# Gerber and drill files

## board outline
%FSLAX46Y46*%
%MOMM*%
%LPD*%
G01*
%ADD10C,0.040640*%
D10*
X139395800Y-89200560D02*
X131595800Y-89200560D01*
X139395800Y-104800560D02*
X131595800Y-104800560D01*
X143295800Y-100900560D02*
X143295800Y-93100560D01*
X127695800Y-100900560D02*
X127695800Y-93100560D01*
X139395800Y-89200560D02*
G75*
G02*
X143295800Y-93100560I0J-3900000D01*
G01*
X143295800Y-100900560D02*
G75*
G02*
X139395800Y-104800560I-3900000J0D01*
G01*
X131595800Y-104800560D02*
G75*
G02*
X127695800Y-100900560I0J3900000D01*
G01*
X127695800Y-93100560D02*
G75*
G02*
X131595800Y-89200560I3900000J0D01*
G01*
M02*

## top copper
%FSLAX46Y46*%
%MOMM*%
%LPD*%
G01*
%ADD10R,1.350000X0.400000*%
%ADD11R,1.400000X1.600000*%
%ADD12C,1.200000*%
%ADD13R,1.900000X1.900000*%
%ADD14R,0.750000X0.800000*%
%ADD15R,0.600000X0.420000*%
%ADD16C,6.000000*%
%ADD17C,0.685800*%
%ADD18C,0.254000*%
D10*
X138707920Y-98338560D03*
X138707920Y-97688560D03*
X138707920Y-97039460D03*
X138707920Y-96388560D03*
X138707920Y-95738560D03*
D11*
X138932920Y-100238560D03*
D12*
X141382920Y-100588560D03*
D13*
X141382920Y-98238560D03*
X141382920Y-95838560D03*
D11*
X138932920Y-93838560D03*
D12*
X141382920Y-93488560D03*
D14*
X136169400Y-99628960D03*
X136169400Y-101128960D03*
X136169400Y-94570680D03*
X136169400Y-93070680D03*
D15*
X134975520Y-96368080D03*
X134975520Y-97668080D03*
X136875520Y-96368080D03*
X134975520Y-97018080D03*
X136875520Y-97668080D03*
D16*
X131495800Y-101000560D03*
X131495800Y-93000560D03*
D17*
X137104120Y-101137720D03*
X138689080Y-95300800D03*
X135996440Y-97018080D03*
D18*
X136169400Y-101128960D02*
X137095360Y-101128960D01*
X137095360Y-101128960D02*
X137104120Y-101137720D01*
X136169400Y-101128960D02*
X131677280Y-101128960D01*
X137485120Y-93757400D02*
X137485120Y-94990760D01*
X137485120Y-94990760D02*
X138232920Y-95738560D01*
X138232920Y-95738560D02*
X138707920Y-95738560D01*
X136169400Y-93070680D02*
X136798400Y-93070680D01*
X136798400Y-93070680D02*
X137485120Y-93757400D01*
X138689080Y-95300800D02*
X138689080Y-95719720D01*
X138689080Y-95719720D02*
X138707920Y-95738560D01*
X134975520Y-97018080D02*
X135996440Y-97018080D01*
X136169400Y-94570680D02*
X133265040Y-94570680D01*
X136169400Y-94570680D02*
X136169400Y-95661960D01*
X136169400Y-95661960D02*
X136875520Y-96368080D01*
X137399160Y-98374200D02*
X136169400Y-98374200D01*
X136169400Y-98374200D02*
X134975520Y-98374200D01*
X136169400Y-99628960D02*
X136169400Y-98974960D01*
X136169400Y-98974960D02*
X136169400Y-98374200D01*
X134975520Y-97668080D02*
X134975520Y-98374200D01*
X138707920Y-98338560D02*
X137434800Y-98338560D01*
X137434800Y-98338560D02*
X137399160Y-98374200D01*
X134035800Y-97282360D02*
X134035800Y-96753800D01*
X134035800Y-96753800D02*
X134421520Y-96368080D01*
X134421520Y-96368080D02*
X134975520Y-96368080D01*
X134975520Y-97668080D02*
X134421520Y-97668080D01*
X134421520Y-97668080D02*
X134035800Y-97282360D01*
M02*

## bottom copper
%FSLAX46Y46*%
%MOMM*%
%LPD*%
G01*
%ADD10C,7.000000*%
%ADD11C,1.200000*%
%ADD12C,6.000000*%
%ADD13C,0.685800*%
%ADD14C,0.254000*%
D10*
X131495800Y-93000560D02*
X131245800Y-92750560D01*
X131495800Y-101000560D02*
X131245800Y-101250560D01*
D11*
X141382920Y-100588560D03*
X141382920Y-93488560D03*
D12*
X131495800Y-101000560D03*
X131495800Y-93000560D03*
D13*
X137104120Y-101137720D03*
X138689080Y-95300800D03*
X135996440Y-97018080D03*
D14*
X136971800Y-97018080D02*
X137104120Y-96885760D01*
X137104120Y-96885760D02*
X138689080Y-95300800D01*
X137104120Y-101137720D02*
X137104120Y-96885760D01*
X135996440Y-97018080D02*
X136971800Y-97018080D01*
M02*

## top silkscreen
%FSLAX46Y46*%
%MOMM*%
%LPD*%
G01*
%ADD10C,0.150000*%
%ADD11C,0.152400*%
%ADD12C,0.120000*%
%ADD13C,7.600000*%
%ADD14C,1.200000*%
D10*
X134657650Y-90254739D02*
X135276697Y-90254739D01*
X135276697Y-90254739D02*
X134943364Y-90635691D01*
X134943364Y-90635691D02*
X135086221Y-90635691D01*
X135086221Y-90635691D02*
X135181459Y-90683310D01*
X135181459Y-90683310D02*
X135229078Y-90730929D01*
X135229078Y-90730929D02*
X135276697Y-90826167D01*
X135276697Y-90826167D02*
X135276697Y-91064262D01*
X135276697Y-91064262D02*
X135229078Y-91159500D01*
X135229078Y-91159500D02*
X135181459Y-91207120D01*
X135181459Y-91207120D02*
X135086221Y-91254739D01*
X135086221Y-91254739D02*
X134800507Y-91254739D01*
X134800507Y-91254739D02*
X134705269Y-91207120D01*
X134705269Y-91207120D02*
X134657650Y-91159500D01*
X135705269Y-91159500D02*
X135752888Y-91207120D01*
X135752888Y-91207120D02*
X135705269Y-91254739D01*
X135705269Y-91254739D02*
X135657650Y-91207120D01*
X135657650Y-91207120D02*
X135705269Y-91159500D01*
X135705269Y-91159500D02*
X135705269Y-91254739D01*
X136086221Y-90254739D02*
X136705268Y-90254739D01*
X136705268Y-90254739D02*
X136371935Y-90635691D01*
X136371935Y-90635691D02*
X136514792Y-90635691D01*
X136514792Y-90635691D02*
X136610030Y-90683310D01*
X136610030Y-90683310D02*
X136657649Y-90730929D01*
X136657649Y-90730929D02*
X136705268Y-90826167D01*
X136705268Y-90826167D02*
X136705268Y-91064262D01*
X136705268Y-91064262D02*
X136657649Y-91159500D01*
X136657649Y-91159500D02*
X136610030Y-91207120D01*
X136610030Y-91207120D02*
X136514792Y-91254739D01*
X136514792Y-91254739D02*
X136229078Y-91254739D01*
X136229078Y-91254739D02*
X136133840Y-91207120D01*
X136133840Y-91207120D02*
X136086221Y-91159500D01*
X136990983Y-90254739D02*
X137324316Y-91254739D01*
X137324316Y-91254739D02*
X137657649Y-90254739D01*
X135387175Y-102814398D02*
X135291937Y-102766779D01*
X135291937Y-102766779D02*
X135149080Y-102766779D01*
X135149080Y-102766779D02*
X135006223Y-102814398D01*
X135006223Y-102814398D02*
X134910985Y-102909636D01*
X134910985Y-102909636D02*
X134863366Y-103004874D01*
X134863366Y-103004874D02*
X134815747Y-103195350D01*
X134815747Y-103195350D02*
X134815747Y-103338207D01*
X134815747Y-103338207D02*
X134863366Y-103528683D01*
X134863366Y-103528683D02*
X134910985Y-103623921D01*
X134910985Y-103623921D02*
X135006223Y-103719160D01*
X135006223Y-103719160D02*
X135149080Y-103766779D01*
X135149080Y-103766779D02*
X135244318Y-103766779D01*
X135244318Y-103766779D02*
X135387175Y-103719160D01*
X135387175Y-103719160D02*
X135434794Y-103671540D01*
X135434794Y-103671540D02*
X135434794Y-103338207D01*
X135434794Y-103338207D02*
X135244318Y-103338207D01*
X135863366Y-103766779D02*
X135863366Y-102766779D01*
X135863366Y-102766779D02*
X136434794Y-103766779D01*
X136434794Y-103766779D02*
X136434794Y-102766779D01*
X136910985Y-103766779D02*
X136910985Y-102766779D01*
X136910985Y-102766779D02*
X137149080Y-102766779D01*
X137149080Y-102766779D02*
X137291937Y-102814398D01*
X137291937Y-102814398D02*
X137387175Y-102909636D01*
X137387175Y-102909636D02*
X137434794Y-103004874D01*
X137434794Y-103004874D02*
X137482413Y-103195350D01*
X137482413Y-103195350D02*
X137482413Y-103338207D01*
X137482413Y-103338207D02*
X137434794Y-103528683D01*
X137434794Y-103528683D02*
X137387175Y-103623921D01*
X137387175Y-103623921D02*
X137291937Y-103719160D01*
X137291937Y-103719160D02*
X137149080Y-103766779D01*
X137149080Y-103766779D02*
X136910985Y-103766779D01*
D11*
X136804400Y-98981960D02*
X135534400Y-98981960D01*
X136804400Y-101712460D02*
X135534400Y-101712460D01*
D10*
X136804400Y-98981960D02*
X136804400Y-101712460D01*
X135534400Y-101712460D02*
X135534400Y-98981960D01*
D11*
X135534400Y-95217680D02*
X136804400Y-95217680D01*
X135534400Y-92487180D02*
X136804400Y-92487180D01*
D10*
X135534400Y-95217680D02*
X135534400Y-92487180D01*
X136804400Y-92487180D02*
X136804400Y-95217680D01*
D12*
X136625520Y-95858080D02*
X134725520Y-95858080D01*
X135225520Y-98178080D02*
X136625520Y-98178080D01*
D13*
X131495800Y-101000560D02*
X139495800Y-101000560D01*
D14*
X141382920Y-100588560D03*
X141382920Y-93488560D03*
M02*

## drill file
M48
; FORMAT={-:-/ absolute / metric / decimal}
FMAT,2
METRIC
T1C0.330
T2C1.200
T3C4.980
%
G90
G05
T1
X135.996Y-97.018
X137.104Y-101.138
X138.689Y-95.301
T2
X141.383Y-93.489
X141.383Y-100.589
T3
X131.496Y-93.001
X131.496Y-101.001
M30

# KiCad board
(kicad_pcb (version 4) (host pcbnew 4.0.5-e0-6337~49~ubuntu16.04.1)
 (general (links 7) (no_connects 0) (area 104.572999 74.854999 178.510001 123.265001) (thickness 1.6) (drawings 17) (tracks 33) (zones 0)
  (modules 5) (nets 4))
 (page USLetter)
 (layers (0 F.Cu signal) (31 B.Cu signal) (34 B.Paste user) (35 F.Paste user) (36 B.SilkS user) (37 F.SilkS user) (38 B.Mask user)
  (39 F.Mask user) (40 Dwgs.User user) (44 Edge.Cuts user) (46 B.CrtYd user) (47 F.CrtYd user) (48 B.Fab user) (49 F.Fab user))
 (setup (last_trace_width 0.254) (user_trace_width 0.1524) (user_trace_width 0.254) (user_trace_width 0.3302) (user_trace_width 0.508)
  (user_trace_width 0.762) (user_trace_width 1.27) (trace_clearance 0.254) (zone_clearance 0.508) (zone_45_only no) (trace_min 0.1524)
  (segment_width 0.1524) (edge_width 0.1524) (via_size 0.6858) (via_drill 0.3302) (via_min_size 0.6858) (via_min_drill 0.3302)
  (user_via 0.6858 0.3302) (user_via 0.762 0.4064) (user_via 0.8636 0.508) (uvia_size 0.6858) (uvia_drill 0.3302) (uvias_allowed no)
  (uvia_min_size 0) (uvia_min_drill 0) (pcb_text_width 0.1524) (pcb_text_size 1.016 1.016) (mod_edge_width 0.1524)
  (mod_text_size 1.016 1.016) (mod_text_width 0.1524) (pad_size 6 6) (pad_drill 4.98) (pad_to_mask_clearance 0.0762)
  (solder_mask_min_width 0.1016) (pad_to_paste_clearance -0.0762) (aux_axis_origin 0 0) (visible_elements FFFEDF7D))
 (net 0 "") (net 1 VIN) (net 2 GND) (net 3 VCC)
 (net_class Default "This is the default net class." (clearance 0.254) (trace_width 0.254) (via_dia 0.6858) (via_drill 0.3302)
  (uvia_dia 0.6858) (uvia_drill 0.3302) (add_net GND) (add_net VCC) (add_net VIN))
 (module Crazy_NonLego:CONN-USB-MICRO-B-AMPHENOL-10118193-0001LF (layer F.Cu) (at 141.38292 97.03856 90)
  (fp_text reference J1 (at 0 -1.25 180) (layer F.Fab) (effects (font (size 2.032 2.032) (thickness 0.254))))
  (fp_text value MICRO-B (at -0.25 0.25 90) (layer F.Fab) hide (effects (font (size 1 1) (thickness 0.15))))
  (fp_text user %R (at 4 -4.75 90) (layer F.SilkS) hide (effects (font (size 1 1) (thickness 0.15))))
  (pad 1 smd rect (at -1.3 -2.675 180) (size 1.35 0.4) (layers F.Cu F.Paste F.Mask) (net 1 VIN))
  (pad 2 smd rect (at -0.65 -2.675 180) (size 1.35 0.4) (layers F.Cu F.Paste F.Mask))
  (pad 3 smd rect (at -0.0009 -2.675 180) (size 1.35 0.4) (layers F.Cu F.Paste F.Mask))
  (pad 4 smd rect (at 0.65 -2.675 180) (size 1.35 0.4) (layers F.Cu F.Paste F.Mask))
  (pad 5 smd rect (at 1.3 -2.675 180) (size 1.35 0.4) (layers F.Cu F.Paste F.Mask) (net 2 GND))
  (pad 6 smd rect (at -3.2 -2.45 180) (size 1.4 1.6) (layers F.Cu F.Paste F.Mask))
  (pad 6 thru_hole circle (at -3.55 0 180) (size 1.2 1.2) (drill 1.2) (layers *.Cu *.Mask F.SilkS))
  (pad 6 smd rect (at -1.2 0 180) (size 1.9 1.9) (layers F.Cu F.Paste F.Mask))
  (pad 6 smd rect (at 1.2 0 180) (size 1.9 1.9) (layers F.Cu F.Paste F.Mask))
  (pad 6 smd rect (at 3.2 -2.45 180) (size 1.4 1.6) (layers F.Cu F.Paste F.Mask))
  (pad 6 thru_hole circle (at 3.55 0 180) (size 1.2 1.2) (drill 1.2) (layers *.Cu *.Mask F.SilkS)))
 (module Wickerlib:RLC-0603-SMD (layer F.Cu) (at 136.1694 100.37896 270)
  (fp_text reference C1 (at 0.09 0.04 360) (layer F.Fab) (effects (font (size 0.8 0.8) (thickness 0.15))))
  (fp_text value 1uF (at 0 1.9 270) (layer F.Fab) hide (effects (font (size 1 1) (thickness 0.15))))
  (fp_line (start -1.397 -0.635) (end -1.397 0.635) (layer F.SilkS) (width 0.1524))
  (fp_line (start 1.3335 -0.635) (end 1.3335 0.635) (layer F.SilkS) (width 0.1524))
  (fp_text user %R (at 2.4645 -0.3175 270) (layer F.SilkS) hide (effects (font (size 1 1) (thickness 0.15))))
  (fp_line (start -1.397 -0.635) (end 1.3335 -0.635) (layer F.SilkS) (width 0.15))
  (fp_line (start 1.3335 0.635) (end -1.397 0.635) (layer F.SilkS) (width 0.15))
  (pad 1 smd rect (at -0.75 0 270) (size 0.8 0.75) (layers F.Cu F.Paste F.Mask) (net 1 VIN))
  (pad 2 smd rect (at 0.75 0 270) (size 0.8 0.75) (layers F.Cu F.Paste F.Mask) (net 2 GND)))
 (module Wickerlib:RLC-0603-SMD (layer F.Cu) (at 136.1694 93.82068 90)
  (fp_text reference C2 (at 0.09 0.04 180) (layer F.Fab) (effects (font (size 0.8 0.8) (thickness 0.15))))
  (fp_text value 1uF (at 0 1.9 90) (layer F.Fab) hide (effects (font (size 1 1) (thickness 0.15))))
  (fp_line (start -1.397 -0.635) (end -1.397 0.635) (layer F.SilkS) (width 0.1524))
  (fp_line (start 1.3335 -0.635) (end 1.3335 0.635) (layer F.SilkS) (width 0.1524))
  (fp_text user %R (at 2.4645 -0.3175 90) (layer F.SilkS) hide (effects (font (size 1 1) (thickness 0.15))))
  (fp_line (start -1.397 -0.635) (end 1.3335 -0.635) (layer F.SilkS) (width 0.15))
  (fp_line (start 1.3335 0.635) (end -1.397 0.635) (layer F.SilkS) (width 0.15))
  (pad 1 smd rect (at -0.75 0 90) (size 0.8 0.75) (layers F.Cu F.Paste F.Mask) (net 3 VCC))
  (pad 2 smd rect (at 0.75 0 90) (size 0.8 0.75) (layers F.Cu F.Paste F.Mask) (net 2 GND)))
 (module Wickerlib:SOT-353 (layer F.Cu) (at 135.92552 97.01808)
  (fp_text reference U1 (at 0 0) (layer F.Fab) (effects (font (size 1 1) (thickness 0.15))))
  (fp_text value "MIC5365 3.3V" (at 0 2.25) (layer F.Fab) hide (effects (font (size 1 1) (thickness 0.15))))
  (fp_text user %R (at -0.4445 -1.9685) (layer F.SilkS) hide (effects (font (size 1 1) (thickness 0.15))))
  (fp_line (start 0.7 -1.16) (end -1.2 -1.16) (layer F.SilkS) (width 0.12))
  (fp_line (start -0.7 1.16) (end 0.7 1.16) (layer F.SilkS) (width 0.12))
  (pad 1 smd rect (at -0.95 -0.65) (size 0.6 0.42) (layers F.Cu F.Paste F.Mask) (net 1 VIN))
  (pad 3 smd rect (at -0.95 0.65) (size 0.6 0.42) (layers F.Cu F.Paste F.Mask) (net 1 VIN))
  (pad 5 smd rect (at 0.95 -0.65) (size 0.6 0.42) (layers F.Cu F.Paste F.Mask) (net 3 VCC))
  (pad 2 smd rect (at -0.95 0) (size 0.6 0.42) (layers F.Cu F.Paste F.Mask) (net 2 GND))
  (pad 4 smd rect (at 0.95 0.65) (size 0.6 0.42) (layers F.Cu F.Paste F.Mask)))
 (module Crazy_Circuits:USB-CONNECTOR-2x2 (layer F.Cu) (at 131.4958 101.00056)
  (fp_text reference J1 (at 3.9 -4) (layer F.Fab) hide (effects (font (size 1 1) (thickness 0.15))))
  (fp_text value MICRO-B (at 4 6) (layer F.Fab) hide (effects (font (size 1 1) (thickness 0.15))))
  (fp_line (start 0 0) (end 8 0) (layer F.SilkS) (width 7.6))
  (fp_line (start 0 -8) (end -0.25 -8.25) (layer B.Cu) (width 7))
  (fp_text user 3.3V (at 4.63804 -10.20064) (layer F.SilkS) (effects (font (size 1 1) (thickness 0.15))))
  (fp_line (start 7.9 -11.8) (end 0.1 -11.8) (layer Edge.Cuts) (width 0.04064))
  (fp_line (start 7.9 3.8) (end 0.1 3.8) (layer Edge.Cuts) (width 0.04064))
  (fp_line (start 11.8 -0.1) (end 11.8 -7.9) (layer Edge.Cuts) (width 0.04064))
  (fp_line (start -3.8 -0.1) (end -3.8 -7.9) (layer Edge.Cuts) (width 0.04064))
  (fp_arc (start 7.9 -7.9) (end 7.9 -11.8) (angle 90) (layer Edge.Cuts) (width 0.04064))
  (fp_arc (start 7.9 -0.1) (end 11.8 -0.1) (angle 90) (layer Edge.Cuts) (width 0.04064))
  (fp_arc (start 0.1 -0.1) (end 0.1 3.8) (angle 90) (layer Edge.Cuts) (width 0.04064))
  (fp_arc (start 0.1 -7.9) (end -3.8 -7.9) (angle 90) (layer Edge.Cuts) (width 0.04064))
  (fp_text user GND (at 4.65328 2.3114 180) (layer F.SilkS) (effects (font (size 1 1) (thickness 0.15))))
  (fp_line (start 0 0) (end -0.25 0.25) (layer B.Cu) (width 7))
  (pad 5 thru_hole circle (at 0 0) (size 6 6) (drill 4.98) (layers *.Cu *.Mask))
  (pad 1 thru_hole circle (at 0 -8) (size 6 6) (drill 4.98) (layers *.Cu *.Mask)))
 (segment (start 136.9718 97.01808) (end 137.10412 96.88576) (width 0.254) (layer B.Cu) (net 2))
 (segment (start 137.10412 96.88576) (end 138.68908 95.3008) (width 0.254) (layer B.Cu) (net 2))
 (segment (start 137.10412 101.13772) (end 137.10412 96.88576) (width 0.254) (layer B.Cu) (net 2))
 (segment (start 136.1694 101.12896) (end 137.09536 101.12896) (width 0.254) (layer F.Cu) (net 2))
 (segment (start 137.09536 101.12896) (end 137.10412 101.13772) (width 0.254) (layer F.Cu) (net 2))
 (via (at 137.10412 101.13772) (size 0.6858) (drill 0.3302) (layers F.Cu B.Cu) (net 2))
 (segment (start 136.1694 101.12896) (end 131.67728 101.12896) (width 0.254) (layer F.Cu) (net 2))
 (segment (start 137.48512 93.7574) (end 137.48512 94.99076) (width 0.254) (layer F.Cu) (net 2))
 (segment (start 137.48512 94.99076) (end 138.23292 95.73856) (width 0.254) (layer F.Cu) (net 2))
 (segment (start 138.23292 95.73856) (end 138.70792 95.73856) (width 0.254) (layer F.Cu) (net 2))
 (segment (start 136.1694 93.07068) (end 136.7984 93.07068) (width 0.254) (layer F.Cu) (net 2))
 (segment (start 136.7984 93.07068) (end 137.48512 93.7574) (width 0.254) (layer F.Cu) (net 2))
 (segment (start 138.68908 95.3008) (end 138.68908 95.71972) (width 0.254) (layer F.Cu) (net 2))
 (segment (start 138.68908 95.71972) (end 138.70792 95.73856) (width 0.254) (layer F.Cu) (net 2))
 (via (at 138.68908 95.3008) (size 0.6858) (drill 0.3302) (layers F.Cu B.Cu) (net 2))
 (segment (start 135.99644 97.01808) (end 136.9718 97.01808) (width 0.254) (layer B.Cu) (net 2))
 (via (at 135.99644 97.01808) (size 0.6858) (drill 0.3302) (layers F.Cu B.Cu) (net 2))
 (segment (start 134.97552 97.01808) (end 135.99644 97.01808) (width 0.254) (layer F.Cu) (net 2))
 (segment (start 136.1694 94.57068) (end 133.26504 94.57068) (width 0.254) (layer F.Cu) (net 3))
 (segment (start 136.1694 94.57068) (end 136.1694 95.66196) (width 0.254) (layer F.Cu) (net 3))
 (segment (start 136.1694 95.66196) (end 136.87552 96.36808) (width 0.254) (layer F.Cu) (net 3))
 (segment (start 137.39916 98.3742) (end 136.1694 98.3742) (width 0.254) (layer F.Cu) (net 1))
 (segment (start 136.1694 98.3742) (end 134.97552 98.3742) (width 0.254) (layer F.Cu) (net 1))
 (segment (start 136.1694 99.62896) (end 136.1694 98.97496) (width 0.254) (layer F.Cu) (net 1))
 (segment (start 136.1694 98.97496) (end 136.1694 98.3742) (width 0.254) (layer F.Cu) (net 1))
 (segment (start 134.97552 97.66808) (end 134.97552 98.3742) (width 0.254) (layer F.Cu) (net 1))
 (segment (start 138.70792 98.33856) (end 137.4348 98.33856) (width 0.254) (layer F.Cu) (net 1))
 (segment (start 137.4348 98.33856) (end 137.39916 98.3742) (width 0.254) (layer F.Cu) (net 1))
 (segment (start 134.0358 97.28236) (end 134.0358 96.7538) (width 0.254) (layer F.Cu) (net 1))
 (segment (start 134.0358 96.7538) (end 134.42152 96.36808) (width 0.254) (layer F.Cu) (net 1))
 (segment (start 134.42152 96.36808) (end 134.97552 96.36808) (width 0.254) (layer F.Cu) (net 1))
 (segment (start 134.97552 97.66808) (end 134.42152 97.66808) (width 0.254) (layer F.Cu) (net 1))
 (segment (start 134.42152 97.66808) (end 134.0358 97.28236) (width 0.254) (layer F.Cu) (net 1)))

